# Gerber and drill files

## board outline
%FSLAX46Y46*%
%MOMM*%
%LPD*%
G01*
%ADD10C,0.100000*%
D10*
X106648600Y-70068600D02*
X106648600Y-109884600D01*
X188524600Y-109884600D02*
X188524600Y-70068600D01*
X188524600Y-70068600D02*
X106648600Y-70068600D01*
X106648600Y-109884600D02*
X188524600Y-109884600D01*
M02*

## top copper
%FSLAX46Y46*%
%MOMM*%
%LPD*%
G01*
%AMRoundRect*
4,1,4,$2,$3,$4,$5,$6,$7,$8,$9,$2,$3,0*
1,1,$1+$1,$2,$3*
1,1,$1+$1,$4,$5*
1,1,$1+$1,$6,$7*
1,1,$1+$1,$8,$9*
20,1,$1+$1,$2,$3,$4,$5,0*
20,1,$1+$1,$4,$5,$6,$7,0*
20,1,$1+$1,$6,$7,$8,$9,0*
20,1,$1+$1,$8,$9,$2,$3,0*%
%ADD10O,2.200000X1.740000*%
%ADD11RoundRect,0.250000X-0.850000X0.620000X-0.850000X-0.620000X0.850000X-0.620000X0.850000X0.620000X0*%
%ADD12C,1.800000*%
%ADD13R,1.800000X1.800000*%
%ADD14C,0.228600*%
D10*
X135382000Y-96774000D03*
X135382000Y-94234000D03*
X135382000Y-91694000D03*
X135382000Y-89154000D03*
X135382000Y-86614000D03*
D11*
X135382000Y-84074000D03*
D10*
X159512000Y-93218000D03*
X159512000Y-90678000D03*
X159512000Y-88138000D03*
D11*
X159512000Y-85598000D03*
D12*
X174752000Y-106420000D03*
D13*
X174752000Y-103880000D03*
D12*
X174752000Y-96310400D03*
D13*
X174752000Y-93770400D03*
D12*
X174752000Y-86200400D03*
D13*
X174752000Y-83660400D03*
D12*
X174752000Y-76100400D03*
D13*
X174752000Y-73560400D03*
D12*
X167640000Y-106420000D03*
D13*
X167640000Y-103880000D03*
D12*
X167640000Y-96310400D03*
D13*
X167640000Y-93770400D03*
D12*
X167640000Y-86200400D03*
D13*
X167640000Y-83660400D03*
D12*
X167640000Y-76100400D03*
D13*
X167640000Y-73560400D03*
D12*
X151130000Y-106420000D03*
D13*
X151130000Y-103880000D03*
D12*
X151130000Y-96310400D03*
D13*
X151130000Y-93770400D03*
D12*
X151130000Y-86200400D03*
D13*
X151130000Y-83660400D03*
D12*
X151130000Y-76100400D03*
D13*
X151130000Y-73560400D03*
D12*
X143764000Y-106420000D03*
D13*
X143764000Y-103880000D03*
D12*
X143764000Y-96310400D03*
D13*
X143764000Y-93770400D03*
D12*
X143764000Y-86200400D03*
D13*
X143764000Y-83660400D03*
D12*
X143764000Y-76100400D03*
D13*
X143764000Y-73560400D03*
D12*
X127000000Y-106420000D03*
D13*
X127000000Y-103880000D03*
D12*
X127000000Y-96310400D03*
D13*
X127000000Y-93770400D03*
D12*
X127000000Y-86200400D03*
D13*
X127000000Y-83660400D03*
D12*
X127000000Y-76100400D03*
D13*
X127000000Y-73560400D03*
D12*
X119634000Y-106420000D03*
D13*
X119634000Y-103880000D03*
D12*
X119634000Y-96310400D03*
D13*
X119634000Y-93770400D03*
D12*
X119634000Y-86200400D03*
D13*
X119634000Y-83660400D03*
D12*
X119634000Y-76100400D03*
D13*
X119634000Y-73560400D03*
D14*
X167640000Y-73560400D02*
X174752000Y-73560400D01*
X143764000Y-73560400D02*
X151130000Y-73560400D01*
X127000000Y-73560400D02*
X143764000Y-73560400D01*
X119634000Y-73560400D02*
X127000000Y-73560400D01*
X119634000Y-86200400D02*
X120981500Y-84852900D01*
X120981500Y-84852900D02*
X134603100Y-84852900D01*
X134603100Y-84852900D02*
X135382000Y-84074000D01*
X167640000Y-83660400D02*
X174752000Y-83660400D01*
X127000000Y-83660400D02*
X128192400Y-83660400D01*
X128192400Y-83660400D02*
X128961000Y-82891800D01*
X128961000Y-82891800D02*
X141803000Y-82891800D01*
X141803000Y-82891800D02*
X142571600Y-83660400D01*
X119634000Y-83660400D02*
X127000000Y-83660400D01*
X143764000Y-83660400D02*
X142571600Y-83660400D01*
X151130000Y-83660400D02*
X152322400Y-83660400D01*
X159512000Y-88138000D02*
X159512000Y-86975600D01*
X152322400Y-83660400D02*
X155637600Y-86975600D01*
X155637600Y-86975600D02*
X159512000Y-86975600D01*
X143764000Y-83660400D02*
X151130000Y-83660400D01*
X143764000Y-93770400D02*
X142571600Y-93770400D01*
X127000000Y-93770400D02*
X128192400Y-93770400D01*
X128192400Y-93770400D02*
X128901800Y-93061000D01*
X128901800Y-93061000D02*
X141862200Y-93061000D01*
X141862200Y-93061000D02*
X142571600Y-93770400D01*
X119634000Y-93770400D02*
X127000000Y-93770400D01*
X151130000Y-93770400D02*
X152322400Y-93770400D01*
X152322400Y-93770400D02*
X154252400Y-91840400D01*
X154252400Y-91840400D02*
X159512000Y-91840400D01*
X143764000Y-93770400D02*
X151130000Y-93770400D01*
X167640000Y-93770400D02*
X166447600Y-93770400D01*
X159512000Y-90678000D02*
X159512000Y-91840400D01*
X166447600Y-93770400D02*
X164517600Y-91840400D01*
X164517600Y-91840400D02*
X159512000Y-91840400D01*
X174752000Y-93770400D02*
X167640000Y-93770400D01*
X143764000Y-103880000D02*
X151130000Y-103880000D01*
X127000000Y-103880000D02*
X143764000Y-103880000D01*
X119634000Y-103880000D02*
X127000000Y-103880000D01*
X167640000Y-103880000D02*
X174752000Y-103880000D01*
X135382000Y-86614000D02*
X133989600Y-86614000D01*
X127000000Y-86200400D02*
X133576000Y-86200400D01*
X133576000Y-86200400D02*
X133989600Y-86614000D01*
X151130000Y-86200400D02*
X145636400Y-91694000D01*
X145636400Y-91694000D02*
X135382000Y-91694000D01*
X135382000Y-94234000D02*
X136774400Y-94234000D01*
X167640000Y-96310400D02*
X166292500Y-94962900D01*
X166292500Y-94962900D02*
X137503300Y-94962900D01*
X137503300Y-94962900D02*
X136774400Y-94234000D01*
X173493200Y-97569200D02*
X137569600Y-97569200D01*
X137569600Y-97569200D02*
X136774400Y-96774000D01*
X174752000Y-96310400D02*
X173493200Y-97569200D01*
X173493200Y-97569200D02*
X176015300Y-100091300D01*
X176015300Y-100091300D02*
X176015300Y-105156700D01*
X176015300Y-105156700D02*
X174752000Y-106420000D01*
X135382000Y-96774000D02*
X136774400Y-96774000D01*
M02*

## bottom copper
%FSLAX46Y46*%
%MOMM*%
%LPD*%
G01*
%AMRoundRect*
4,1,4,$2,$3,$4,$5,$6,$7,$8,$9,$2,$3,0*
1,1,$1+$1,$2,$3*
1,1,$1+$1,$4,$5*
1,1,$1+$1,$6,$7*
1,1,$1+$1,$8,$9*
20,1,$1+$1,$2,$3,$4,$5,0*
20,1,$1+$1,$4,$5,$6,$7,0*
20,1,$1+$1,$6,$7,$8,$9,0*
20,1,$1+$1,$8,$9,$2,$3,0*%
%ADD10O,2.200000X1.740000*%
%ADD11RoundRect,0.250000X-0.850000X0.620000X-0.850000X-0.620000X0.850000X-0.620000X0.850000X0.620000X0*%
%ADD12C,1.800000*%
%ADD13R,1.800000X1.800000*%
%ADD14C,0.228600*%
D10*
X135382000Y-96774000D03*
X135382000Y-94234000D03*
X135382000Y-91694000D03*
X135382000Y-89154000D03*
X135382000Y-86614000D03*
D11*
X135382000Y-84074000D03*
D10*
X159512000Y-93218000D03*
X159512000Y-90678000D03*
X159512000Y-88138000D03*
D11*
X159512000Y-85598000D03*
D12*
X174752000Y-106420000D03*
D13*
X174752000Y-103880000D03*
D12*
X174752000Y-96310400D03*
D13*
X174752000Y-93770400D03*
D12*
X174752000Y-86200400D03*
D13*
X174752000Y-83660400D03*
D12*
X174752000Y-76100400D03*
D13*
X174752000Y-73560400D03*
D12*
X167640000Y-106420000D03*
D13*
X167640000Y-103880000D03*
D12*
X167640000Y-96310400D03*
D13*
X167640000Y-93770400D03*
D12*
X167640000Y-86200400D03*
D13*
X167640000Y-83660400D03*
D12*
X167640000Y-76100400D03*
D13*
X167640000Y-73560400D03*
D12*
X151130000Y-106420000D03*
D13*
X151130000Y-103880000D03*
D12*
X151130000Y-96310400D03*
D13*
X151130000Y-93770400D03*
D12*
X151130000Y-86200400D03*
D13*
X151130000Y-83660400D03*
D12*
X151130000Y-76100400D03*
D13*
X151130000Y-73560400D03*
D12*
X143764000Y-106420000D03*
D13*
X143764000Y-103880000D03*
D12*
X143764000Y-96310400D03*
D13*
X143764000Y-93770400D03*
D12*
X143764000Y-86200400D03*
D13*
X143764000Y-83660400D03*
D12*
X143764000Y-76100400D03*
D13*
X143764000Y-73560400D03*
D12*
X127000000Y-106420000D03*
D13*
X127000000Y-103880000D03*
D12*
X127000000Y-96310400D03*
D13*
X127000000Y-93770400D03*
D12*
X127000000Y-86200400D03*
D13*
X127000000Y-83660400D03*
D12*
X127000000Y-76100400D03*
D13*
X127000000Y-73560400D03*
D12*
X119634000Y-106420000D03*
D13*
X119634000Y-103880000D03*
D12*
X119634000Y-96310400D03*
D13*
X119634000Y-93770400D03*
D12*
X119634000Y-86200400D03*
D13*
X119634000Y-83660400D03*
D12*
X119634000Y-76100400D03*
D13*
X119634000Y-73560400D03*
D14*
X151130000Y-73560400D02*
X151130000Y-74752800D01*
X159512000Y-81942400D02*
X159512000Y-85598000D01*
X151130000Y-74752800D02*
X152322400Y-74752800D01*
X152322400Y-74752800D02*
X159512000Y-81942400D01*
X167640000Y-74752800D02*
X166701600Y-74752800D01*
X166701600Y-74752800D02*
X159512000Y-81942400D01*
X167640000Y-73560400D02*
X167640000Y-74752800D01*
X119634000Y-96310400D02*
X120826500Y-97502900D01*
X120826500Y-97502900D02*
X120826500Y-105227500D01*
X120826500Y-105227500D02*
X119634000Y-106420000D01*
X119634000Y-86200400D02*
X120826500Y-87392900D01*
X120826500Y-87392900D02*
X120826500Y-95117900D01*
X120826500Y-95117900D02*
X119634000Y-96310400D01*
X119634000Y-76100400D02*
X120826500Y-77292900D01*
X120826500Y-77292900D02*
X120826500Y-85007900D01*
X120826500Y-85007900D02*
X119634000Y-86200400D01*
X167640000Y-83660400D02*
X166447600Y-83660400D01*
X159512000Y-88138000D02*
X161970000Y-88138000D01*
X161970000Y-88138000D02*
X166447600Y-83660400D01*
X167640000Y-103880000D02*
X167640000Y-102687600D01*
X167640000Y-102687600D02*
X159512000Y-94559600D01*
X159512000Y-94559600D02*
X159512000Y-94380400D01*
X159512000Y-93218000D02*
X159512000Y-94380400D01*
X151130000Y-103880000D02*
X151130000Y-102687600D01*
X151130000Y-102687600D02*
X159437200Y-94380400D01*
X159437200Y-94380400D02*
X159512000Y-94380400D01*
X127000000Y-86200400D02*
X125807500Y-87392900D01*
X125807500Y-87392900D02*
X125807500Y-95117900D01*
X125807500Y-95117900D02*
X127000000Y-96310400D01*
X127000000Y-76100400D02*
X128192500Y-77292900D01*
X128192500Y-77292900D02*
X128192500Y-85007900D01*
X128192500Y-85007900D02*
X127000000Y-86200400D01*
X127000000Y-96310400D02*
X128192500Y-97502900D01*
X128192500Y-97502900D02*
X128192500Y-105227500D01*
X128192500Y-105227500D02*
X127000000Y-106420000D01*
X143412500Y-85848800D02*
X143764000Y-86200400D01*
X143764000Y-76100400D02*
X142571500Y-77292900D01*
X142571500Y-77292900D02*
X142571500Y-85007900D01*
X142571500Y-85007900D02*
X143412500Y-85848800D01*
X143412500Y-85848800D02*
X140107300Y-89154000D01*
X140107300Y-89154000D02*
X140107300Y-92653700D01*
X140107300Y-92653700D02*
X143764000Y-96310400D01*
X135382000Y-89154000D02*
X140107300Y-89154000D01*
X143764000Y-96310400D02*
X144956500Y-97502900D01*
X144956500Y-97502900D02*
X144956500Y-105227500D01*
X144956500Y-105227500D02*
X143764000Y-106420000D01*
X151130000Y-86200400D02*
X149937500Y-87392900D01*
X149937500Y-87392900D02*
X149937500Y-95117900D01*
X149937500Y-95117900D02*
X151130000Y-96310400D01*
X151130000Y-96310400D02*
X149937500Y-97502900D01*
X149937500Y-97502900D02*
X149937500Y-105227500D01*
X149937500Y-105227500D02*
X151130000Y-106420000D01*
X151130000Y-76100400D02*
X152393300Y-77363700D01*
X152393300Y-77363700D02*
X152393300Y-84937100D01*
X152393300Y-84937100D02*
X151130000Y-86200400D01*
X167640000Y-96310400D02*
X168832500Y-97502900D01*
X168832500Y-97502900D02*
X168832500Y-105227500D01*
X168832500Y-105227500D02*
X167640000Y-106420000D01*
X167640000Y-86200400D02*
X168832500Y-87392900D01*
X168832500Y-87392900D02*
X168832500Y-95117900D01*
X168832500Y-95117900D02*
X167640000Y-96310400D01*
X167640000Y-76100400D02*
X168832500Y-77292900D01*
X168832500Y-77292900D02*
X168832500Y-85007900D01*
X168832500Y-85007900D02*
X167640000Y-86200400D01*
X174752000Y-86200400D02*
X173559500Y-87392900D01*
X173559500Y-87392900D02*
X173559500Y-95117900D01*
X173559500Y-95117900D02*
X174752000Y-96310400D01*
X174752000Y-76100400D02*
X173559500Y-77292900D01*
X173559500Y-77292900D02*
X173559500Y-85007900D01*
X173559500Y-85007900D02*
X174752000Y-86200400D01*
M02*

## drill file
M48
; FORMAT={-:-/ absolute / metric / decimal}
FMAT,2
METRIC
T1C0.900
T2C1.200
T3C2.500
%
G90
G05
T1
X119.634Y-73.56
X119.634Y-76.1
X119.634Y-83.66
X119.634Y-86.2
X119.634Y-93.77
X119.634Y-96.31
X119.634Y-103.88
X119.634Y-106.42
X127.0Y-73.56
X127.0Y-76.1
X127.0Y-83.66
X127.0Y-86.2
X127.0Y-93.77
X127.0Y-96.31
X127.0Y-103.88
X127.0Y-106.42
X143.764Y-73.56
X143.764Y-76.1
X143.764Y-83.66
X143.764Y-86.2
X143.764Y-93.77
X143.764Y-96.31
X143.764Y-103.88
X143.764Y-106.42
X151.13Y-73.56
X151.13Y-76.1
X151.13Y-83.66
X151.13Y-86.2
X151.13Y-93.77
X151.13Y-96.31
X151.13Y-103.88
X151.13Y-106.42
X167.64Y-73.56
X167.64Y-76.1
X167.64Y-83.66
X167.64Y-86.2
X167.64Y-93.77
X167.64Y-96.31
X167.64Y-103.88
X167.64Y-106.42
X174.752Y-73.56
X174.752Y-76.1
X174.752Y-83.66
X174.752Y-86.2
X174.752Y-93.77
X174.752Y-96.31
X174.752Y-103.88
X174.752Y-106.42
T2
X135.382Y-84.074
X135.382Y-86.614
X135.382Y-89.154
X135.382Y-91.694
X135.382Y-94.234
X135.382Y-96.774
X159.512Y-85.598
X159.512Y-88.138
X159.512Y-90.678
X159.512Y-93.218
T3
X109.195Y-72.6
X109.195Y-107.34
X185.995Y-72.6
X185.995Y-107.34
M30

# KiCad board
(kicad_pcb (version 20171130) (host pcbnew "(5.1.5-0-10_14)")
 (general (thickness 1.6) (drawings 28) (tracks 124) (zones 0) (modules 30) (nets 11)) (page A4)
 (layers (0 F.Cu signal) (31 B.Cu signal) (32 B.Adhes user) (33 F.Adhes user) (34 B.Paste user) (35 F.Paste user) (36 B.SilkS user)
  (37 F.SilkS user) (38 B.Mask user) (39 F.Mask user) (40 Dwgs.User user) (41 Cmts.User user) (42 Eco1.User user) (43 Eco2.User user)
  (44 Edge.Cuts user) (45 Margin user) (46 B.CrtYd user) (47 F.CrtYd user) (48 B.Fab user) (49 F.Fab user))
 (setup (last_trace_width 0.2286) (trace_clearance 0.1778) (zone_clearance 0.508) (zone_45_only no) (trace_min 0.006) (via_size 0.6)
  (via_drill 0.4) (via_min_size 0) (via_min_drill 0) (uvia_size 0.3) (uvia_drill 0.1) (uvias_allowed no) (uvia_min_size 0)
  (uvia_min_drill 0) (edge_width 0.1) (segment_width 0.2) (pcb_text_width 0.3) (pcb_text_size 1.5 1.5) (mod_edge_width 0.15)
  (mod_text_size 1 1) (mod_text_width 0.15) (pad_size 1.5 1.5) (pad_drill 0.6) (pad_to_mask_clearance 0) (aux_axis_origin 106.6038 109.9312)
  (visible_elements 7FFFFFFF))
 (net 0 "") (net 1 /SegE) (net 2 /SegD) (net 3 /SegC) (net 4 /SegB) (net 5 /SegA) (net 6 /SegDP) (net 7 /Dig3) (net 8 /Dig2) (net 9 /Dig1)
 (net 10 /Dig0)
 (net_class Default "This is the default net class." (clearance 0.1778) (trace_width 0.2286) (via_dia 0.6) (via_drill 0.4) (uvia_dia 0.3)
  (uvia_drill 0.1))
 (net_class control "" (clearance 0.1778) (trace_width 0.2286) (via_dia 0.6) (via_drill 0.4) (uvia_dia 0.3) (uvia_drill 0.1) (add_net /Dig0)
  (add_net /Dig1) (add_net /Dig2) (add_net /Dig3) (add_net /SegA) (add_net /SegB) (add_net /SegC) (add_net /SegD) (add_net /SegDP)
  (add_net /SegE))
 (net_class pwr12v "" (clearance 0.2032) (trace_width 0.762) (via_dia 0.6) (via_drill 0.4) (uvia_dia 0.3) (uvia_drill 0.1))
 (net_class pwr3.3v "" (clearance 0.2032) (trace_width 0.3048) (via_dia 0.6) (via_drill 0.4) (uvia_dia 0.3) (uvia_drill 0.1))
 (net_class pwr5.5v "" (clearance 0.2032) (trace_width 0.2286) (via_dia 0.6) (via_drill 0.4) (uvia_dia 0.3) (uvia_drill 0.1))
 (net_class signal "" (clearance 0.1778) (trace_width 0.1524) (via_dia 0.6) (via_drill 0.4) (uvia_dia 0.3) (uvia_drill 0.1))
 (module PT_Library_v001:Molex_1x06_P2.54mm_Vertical (layer B.Cu) (at 135.382 84.074 270)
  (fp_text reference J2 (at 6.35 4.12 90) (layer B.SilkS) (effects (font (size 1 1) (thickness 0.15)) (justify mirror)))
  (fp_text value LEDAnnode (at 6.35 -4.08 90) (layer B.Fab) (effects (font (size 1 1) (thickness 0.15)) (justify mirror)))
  (pad 6 thru_hole oval (at 12.7 0 270) (size 1.74 2.2) (drill 1.2) (layers *.Cu *.Mask) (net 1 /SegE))
  (pad 5 thru_hole oval (at 10.16 0 270) (size 1.74 2.2) (drill 1.2) (layers *.Cu *.Mask) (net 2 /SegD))
  (pad 4 thru_hole oval (at 7.62 0 270) (size 1.74 2.2) (drill 1.2) (layers *.Cu *.Mask) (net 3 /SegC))
  (pad 3 thru_hole oval (at 5.08 0 270) (size 1.74 2.2) (drill 1.2) (layers *.Cu *.Mask) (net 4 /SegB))
  (pad 2 thru_hole oval (at 2.54 0 270) (size 1.74 2.2) (drill 1.2) (layers *.Cu *.Mask) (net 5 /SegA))
  (pad 1 thru_hole roundrect (at 0 0 270) (size 1.74 2.2) (drill 1.2) (layers *.Cu *.Mask) (roundrect_rratio 0.143678) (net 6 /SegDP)))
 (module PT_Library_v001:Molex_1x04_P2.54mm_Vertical (layer B.Cu) (at 159.512 85.598 270)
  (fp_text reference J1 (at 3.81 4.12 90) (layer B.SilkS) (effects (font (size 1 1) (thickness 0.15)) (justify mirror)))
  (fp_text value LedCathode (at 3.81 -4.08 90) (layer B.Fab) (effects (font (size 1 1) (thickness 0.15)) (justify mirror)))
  (pad 4 thru_hole oval (at 7.62 0 270) (size 1.74 2.2) (drill 1.2) (layers *.Cu *.Mask) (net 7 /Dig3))
  (pad 3 thru_hole oval (at 5.08 0 270) (size 1.74 2.2) (drill 1.2) (layers *.Cu *.Mask) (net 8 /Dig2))
  (pad 2 thru_hole oval (at 2.54 0 270) (size 1.74 2.2) (drill 1.2) (layers *.Cu *.Mask) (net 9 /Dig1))
  (pad 1 thru_hole roundrect (at 0 0 270) (size 1.74 2.2) (drill 1.2) (layers *.Cu *.Mask) (roundrect_rratio 0.143678) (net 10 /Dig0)))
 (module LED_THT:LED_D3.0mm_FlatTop (layer F.Cu) (at 174.752 103.88 270)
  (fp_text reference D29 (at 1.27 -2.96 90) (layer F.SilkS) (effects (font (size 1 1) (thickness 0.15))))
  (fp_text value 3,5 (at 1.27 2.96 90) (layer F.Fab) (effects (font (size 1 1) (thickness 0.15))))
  (pad 2 thru_hole circle (at 2.54 0 270) (size 1.8 1.8) (drill 0.9) (layers *.Cu *.Mask) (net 1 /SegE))
  (pad 1 thru_hole rect (at 0 0 270) (size 1.8 1.8) (drill 0.9) (layers *.Cu *.Mask) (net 7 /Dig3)))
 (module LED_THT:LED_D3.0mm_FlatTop (layer F.Cu) (at 174.752 93.7704 270)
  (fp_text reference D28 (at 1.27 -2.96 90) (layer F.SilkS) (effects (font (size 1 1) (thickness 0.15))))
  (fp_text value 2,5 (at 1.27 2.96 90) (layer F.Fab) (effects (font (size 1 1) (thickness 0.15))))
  (pad 2 thru_hole circle (at 2.54 0 270) (size 1.8 1.8) (drill 0.9) (layers *.Cu *.Mask) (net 1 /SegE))
  (pad 1 thru_hole rect (at 0 0 270) (size 1.8 1.8) (drill 0.9) (layers *.Cu *.Mask) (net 8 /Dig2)))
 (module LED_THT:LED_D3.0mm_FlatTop (layer F.Cu) (at 174.752 83.6604 270)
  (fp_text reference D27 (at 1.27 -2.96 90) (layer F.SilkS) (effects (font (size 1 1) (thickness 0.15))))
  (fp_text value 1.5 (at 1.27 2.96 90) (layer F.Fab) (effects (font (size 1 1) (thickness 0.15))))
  (pad 2 thru_hole circle (at 2.54 0 270) (size 1.8 1.8) (drill 0.9) (layers *.Cu *.Mask) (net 1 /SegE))
  (pad 1 thru_hole rect (at 0 0 270) (size 1.8 1.8) (drill 0.9) (layers *.Cu *.Mask) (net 9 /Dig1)))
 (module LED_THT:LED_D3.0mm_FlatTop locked (layer F.Cu) (at 174.752 73.5604 270)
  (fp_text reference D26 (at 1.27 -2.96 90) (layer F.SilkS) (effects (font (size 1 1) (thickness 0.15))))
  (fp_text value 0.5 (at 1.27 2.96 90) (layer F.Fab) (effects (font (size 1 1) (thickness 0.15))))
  (pad 2 thru_hole circle (at 2.54 0 270) (size 1.8 1.8) (drill 0.9) (layers *.Cu *.Mask) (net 1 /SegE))
  (pad 1 thru_hole rect (at 0 0 270) (size 1.8 1.8) (drill 0.9) (layers *.Cu *.Mask) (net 10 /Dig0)))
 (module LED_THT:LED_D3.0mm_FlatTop (layer F.Cu) (at 167.64 103.88 270)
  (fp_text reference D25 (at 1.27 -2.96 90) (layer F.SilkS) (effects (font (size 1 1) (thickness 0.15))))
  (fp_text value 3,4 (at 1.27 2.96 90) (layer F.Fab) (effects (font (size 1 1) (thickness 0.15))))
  (pad 2 thru_hole circle (at 2.54 0 270) (size 1.8 1.8) (drill 0.9) (layers *.Cu *.Mask) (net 2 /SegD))
  (pad 1 thru_hole rect (at 0 0 270) (size 1.8 1.8) (drill 0.9) (layers *.Cu *.Mask) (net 7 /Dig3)))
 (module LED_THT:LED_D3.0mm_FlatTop (layer F.Cu) (at 167.64 93.7704 270)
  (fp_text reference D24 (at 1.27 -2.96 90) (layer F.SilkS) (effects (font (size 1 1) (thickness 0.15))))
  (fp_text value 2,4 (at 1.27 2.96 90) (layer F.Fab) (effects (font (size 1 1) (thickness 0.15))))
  (pad 2 thru_hole circle (at 2.54 0 270) (size 1.8 1.8) (drill 0.9) (layers *.Cu *.Mask) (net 2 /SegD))
  (pad 1 thru_hole rect (at 0 0 270) (size 1.8 1.8) (drill 0.9) (layers *.Cu *.Mask) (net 8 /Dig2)))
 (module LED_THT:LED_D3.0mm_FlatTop (layer F.Cu) (at 167.64 83.6604 270)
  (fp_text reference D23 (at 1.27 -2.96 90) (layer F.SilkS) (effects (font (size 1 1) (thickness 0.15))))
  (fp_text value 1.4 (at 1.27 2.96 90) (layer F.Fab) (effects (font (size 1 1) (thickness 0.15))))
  (pad 2 thru_hole circle (at 2.54 0 270) (size 1.8 1.8) (drill 0.9) (layers *.Cu *.Mask) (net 2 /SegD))
  (pad 1 thru_hole rect (at 0 0 270) (size 1.8 1.8) (drill 0.9) (layers *.Cu *.Mask) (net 9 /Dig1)))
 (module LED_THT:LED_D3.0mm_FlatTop (layer F.Cu) (at 167.64 73.5604 270)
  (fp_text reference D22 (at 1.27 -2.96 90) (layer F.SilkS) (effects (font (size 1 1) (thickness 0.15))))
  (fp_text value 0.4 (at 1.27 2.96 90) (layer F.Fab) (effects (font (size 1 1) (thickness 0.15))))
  (pad 2 thru_hole circle (at 2.54 0 270) (size 1.8 1.8) (drill 0.9) (layers *.Cu *.Mask) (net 2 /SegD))
  (pad 1 thru_hole rect (at 0 0 270) (size 1.8 1.8) (drill 0.9) (layers *.Cu *.Mask) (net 10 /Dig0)))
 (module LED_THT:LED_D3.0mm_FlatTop (layer F.Cu) (at 151.13 103.88 270)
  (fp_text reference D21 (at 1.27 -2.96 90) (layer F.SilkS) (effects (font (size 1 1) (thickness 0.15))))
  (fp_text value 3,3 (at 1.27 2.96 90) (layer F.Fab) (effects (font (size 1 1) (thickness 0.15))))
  (pad 2 thru_hole circle (at 2.54 0 270) (size 1.8 1.8) (drill 0.9) (layers *.Cu *.Mask) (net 3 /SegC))
  (pad 1 thru_hole rect (at 0 0 270) (size 1.8 1.8) (drill 0.9) (layers *.Cu *.Mask) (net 7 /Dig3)))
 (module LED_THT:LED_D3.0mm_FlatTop (layer F.Cu) (at 151.13 93.7704 270)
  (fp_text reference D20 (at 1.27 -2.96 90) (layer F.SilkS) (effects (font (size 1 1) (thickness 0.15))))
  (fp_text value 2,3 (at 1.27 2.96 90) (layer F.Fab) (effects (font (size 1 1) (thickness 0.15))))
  (pad 2 thru_hole circle (at 2.54 0 270) (size 1.8 1.8) (drill 0.9) (layers *.Cu *.Mask) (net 3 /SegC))
  (pad 1 thru_hole rect (at 0 0 270) (size 1.8 1.8) (drill 0.9) (layers *.Cu *.Mask) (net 8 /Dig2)))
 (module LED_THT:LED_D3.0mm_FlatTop (layer F.Cu) (at 151.13 83.6604 270)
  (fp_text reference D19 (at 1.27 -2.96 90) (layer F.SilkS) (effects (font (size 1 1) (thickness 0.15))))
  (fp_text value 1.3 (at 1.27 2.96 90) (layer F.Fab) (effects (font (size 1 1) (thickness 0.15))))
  (pad 2 thru_hole circle (at 2.54 0 270) (size 1.8 1.8) (drill 0.9) (layers *.Cu *.Mask) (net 3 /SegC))
  (pad 1 thru_hole rect (at 0 0 270) (size 1.8 1.8) (drill 0.9) (layers *.Cu *.Mask) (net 9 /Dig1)))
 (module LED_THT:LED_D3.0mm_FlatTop (layer F.Cu) (at 151.13 73.5604 270)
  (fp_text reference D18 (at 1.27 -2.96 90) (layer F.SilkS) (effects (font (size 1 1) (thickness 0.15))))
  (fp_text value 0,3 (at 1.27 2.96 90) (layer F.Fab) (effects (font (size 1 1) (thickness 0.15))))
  (pad 2 thru_hole circle (at 2.54 0 270) (size 1.8 1.8) (drill 0.9) (layers *.Cu *.Mask) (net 3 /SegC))
  (pad 1 thru_hole rect (at 0 0 270) (size 1.8 1.8) (drill 0.9) (layers *.Cu *.Mask) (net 10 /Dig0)))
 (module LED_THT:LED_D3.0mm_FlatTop (layer F.Cu) (at 143.764 103.88 270)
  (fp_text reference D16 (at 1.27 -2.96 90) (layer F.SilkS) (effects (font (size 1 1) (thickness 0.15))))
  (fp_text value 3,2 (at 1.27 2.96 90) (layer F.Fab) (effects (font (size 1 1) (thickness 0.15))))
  (pad 2 thru_hole circle (at 2.54 0 270) (size 1.8 1.8) (drill 0.9) (layers *.Cu *.Mask) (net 4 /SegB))
  (pad 1 thru_hole rect (at 0 0 270) (size 1.8 1.8) (drill 0.9) (layers *.Cu *.Mask) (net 7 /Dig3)))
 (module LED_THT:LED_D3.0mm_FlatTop (layer F.Cu) (at 143.764 93.7704 270)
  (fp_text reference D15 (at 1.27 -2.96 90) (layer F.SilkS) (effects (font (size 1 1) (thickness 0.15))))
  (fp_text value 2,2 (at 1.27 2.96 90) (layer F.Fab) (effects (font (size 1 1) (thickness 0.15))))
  (pad 2 thru_hole circle (at 2.54 0 270) (size 1.8 1.8) (drill 0.9) (layers *.Cu *.Mask) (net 4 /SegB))
  (pad 1 thru_hole rect (at 0 0 270) (size 1.8 1.8) (drill 0.9) (layers *.Cu *.Mask) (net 8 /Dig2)))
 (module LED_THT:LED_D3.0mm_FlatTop (layer F.Cu) (at 143.764 83.6604 270)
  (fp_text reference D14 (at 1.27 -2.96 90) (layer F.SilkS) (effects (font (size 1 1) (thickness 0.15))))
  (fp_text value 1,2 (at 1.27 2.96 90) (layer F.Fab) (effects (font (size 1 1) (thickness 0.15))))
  (pad 2 thru_hole circle (at 2.54 0 270) (size 1.8 1.8) (drill 0.9) (layers *.Cu *.Mask) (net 4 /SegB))
  (pad 1 thru_hole rect (at 0 0 270) (size 1.8 1.8) (drill 0.9) (layers *.Cu *.Mask) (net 9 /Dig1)))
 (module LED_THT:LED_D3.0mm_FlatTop (layer F.Cu) (at 143.764 73.5604 270)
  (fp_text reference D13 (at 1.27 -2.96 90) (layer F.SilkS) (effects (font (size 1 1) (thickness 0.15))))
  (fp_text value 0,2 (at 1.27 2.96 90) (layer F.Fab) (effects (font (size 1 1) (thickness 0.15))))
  (pad 2 thru_hole circle (at 2.54 0 270) (size 1.8 1.8) (drill 0.9) (layers *.Cu *.Mask) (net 4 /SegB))
  (pad 1 thru_hole rect (at 0 0 270) (size 1.8 1.8) (drill 0.9) (layers *.Cu *.Mask) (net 10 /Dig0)))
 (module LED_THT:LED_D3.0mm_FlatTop (layer F.Cu) (at 127 103.88 270)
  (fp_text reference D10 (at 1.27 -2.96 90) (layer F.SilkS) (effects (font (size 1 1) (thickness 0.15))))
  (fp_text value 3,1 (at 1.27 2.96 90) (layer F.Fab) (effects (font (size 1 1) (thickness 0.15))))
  (pad 2 thru_hole circle (at 2.54 0 270) (size 1.8 1.8) (drill 0.9) (layers *.Cu *.Mask) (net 5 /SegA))
  (pad 1 thru_hole rect (at 0 0 270) (size 1.8 1.8) (drill 0.9) (layers *.Cu *.Mask) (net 7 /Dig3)))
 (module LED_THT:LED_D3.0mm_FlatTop (layer F.Cu) (at 127 93.7704 270)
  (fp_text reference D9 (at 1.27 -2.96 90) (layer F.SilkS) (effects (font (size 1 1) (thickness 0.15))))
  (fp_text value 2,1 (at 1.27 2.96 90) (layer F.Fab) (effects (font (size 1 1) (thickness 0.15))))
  (pad 2 thru_hole circle (at 2.54 0 270) (size 1.8 1.8) (drill 0.9) (layers *.Cu *.Mask) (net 5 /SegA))
  (pad 1 thru_hole rect (at 0 0 270) (size 1.8 1.8) (drill 0.9) (layers *.Cu *.Mask) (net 8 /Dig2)))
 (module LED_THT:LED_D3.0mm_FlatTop (layer F.Cu) (at 127 83.6604 270)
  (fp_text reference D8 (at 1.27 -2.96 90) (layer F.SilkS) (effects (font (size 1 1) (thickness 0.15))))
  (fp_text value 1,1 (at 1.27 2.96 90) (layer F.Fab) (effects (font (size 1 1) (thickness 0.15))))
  (pad 2 thru_hole circle (at 2.54 0 270) (size 1.8 1.8) (drill 0.9) (layers *.Cu *.Mask) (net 5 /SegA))
  (pad 1 thru_hole rect (at 0 0 270) (size 1.8 1.8) (drill 0.9) (layers *.Cu *.Mask) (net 9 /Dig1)))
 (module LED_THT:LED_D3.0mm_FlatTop (layer F.Cu) (at 127 73.5604 270)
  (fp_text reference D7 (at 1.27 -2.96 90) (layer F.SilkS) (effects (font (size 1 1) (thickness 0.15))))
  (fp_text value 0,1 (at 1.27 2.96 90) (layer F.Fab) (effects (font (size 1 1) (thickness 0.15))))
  (pad 2 thru_hole circle (at 2.54 0 270) (size 1.8 1.8) (drill 0.9) (layers *.Cu *.Mask) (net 5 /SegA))
  (pad 1 thru_hole rect (at 0 0 270) (size 1.8 1.8) (drill 0.9) (layers *.Cu *.Mask) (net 10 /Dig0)))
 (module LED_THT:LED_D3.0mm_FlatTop (layer F.Cu) (at 119.634 103.88 270)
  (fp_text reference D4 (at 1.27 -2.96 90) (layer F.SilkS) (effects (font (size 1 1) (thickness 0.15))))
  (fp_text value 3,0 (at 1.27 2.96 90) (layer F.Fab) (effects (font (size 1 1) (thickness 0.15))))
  (pad 2 thru_hole circle (at 2.54 0 270) (size 1.8 1.8) (drill 0.9) (layers *.Cu *.Mask) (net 6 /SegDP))
  (pad 1 thru_hole rect (at 0 0 270) (size 1.8 1.8) (drill 0.9) (layers *.Cu *.Mask) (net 7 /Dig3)))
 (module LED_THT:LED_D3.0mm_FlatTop (layer F.Cu) (at 119.634 93.7704 270)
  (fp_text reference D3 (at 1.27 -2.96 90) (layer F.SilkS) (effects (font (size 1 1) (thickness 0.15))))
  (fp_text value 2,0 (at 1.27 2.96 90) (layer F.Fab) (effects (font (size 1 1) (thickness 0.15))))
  (pad 2 thru_hole circle (at 2.54 0 270) (size 1.8 1.8) (drill 0.9) (layers *.Cu *.Mask) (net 6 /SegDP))
  (pad 1 thru_hole rect (at 0 0 270) (size 1.8 1.8) (drill 0.9) (layers *.Cu *.Mask) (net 8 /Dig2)))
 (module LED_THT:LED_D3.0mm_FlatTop (layer F.Cu) (at 119.634 83.6604 270)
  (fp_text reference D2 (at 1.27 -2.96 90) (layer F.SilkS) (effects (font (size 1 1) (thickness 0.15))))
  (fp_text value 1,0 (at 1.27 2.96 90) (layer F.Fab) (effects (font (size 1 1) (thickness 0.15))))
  (pad 2 thru_hole circle (at 2.54 0 270) (size 1.8 1.8) (drill 0.9) (layers *.Cu *.Mask) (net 6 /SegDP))
  (pad 1 thru_hole rect (at 0 0 270) (size 1.8 1.8) (drill 0.9) (layers *.Cu *.Mask) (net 9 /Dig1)))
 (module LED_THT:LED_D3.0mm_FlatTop (layer F.Cu) (at 119.634 73.5604 270)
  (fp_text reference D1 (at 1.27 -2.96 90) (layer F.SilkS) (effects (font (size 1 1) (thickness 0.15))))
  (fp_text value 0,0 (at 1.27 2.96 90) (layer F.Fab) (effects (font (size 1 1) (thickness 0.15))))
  (pad 2 thru_hole circle (at 2.54 0 270) (size 1.8 1.8) (drill 0.9) (layers *.Cu *.Mask) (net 6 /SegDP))
  (pad 1 thru_hole rect (at 0 0 270) (size 1.8 1.8) (drill 0.9) (layers *.Cu *.Mask) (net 10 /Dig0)))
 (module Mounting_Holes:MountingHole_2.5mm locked (layer F.Cu) (at 109.195 72.6004)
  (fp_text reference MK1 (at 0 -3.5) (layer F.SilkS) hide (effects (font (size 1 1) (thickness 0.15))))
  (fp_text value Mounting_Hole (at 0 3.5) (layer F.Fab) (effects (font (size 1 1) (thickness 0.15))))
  (pad 1 np_thru_hole circle (at 0 0) (size 2.5 2.5) (drill 2.5) (layers *.Cu *.Mask)))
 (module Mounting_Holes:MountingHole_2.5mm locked (layer F.Cu) (at 185.995 72.6004)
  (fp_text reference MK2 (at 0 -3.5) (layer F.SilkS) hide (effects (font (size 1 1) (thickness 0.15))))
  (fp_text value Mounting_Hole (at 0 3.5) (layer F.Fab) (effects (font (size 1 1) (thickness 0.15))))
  (pad 1 np_thru_hole circle (at 0 0) (size 2.5 2.5) (drill 2.5) (layers *.Cu *.Mask)))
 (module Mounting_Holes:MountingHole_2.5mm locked (layer F.Cu) (at 109.195 107.34)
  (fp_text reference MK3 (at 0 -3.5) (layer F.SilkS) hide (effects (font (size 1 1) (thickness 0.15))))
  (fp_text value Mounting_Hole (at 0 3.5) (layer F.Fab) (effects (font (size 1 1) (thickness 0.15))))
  (pad 1 np_thru_hole circle (at 0 0) (size 2.5 2.5) (drill 2.5) (layers *.Cu *.Mask)))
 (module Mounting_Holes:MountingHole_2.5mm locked (layer F.Cu) (at 185.995 107.34)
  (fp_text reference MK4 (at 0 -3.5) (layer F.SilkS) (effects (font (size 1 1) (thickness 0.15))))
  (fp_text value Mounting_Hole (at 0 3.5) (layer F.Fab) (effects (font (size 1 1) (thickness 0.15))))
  (pad 1 np_thru_hole circle (at 0 0) (size 2.5 2.5) (drill 2.5) (layers *.Cu *.Mask)))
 (gr_line (start 106.6486 70.0686) (end 106.6486 109.8846) (layer Edge.Cuts) (width 0.1))
 (gr_line (start 188.5246 109.8846) (end 188.5246 70.0686) (layer Edge.Cuts) (width 0.1))
 (gr_line (start 188.5246 70.0686) (end 106.6486 70.0686) (layer Edge.Cuts) (width 0.1))
 (gr_line (start 106.6486 109.8846) (end 188.5246 109.8846) (layer Edge.Cuts) (width 0.1))
 (segment (start 151.13 73.5604) (end 151.13 74.7528) (width 0.2286) (layer B.Cu) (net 10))
 (segment (start 159.512 81.9424) (end 159.512 85.598) (width 0.2286) (layer B.Cu) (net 10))
 (segment (start 151.13 74.7528) (end 152.3224 74.7528) (width 0.2286) (layer B.Cu) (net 10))
 (segment (start 152.3224 74.7528) (end 159.512 81.9424) (width 0.2286) (layer B.Cu) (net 10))
 (segment (start 167.64 74.7528) (end 166.7016 74.7528) (width 0.2286) (layer B.Cu) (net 10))
 (segment (start 166.7016 74.7528) (end 159.512 81.9424) (width 0.2286) (layer B.Cu) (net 10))
 (segment (start 167.64 73.5604) (end 167.64 74.7528) (width 0.2286) (layer B.Cu) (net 10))
 (segment (start 167.64 73.5604) (end 174.752 73.5604) (width 0.2286) (layer F.Cu) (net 10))
 (segment (start 143.764 73.5604) (end 151.13 73.5604) (width 0.2286) (layer F.Cu) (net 10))
 (segment (start 127 73.5604) (end 143.764 73.5604) (width 0.2286) (layer F.Cu) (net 10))
 (segment (start 119.634 73.5604) (end 127 73.5604) (width 0.2286) (layer F.Cu) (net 10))
 (segment (start 119.634 86.2004) (end 120.9815 84.8529) (width 0.2286) (layer F.Cu) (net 6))
 (segment (start 120.9815 84.8529) (end 134.6031 84.8529) (width 0.2286) (layer F.Cu) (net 6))
 (segment (start 134.6031 84.8529) (end 135.382 84.074) (width 0.2286) (layer F.Cu) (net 6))
 (segment (start 119.634 96.3104) (end 120.8265 97.5029) (width 0.2286) (layer B.Cu) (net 6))
 (segment (start 120.8265 97.5029) (end 120.8265 105.2275) (width 0.2286) (layer B.Cu) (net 6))
 (segment (start 120.8265 105.2275) (end 119.634 106.42) (width 0.2286) (layer B.Cu) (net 6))
 (segment (start 119.634 86.2004) (end 120.8265 87.3929) (width 0.2286) (layer B.Cu) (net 6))
 (segment (start 120.8265 87.3929) (end 120.8265 95.1179) (width 0.2286) (layer B.Cu) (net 6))
 (segment (start 120.8265 95.1179) (end 119.634 96.3104) (width 0.2286) (layer B.Cu) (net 6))
 (segment (start 119.634 76.1004) (end 120.8265 77.2929) (width 0.2286) (layer B.Cu) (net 6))
 (segment (start 120.8265 77.2929) (end 120.8265 85.0079) (width 0.2286) (layer B.Cu) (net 6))
 (segment (start 120.8265 85.0079) (end 119.634 86.2004) (width 0.2286) (layer B.Cu) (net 6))
 (segment (start 167.64 83.6604) (end 174.752 83.6604) (width 0.2286) (layer F.Cu) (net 9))
 (segment (start 167.64 83.6604) (end 166.4476 83.6604) (width 0.2286) (layer B.Cu) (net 9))
 (segment (start 159.512 88.138) (end 161.97 88.138) (width 0.2286) (layer B.Cu) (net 9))
 (segment (start 161.97 88.138) (end 166.4476 83.6604) (width 0.2286) (layer B.Cu) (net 9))
 (segment (start 127 83.6604) (end 128.1924 83.6604) (width 0.2286) (layer F.Cu) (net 9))
 (segment (start 128.1924 83.6604) (end 128.961 82.8918) (width 0.2286) (layer F.Cu) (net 9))
 (segment (start 128.961 82.8918) (end 141.803 82.8918) (width 0.2286) (layer F.Cu) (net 9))
 (segment (start 141.803 82.8918) (end 142.5716 83.6604) (width 0.2286) (layer F.Cu) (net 9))
 (segment (start 119.634 83.6604) (end 127 83.6604) (width 0.2286) (layer F.Cu) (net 9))
 (segment (start 143.764 83.6604) (end 142.5716 83.6604) (width 0.2286) (layer F.Cu) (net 9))
 (segment (start 151.13 83.6604) (end 152.3224 83.6604) (width 0.2286) (layer F.Cu) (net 9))
 (segment (start 159.512 88.138) (end 159.512 86.9756) (width 0.2286) (layer F.Cu) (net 9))
 (segment (start 152.3224 83.6604) (end 155.6376 86.9756) (width 0.2286) (layer F.Cu) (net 9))
 (segment (start 155.6376 86.9756) (end 159.512 86.9756) (width 0.2286) (layer F.Cu) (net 9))
 (segment (start 143.764 83.6604) (end 151.13 83.6604) (width 0.2286) (layer F.Cu) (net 9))
 (segment (start 143.764 93.7704) (end 142.5716 93.7704) (width 0.2286) (layer F.Cu) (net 8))
 (segment (start 127 93.7704) (end 128.1924 93.7704) (width 0.2286) (layer F.Cu) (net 8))
 (segment (start 128.1924 93.7704) (end 128.9018 93.061) (width 0.2286) (layer F.Cu) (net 8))
 (segment (start 128.9018 93.061) (end 141.8622 93.061) (width 0.2286) (layer F.Cu) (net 8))
 (segment (start 141.8622 93.061) (end 142.5716 93.7704) (width 0.2286) (layer F.Cu) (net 8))
 (segment (start 119.634 93.7704) (end 127 93.7704) (width 0.2286) (layer F.Cu) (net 8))
 (segment (start 151.13 93.7704) (end 152.3224 93.7704) (width 0.2286) (layer F.Cu) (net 8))
 (segment (start 152.3224 93.7704) (end 154.2524 91.8404) (width 0.2286) (layer F.Cu) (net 8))
 (segment (start 154.2524 91.8404) (end 159.512 91.8404) (width 0.2286) (layer F.Cu) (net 8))
 (segment (start 143.764 93.7704) (end 151.13 93.7704) (width 0.2286) (layer F.Cu) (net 8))
 (segment (start 167.64 93.7704) (end 166.4476 93.7704) (width 0.2286) (layer F.Cu) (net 8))
 (segment (start 159.512 90.678) (end 159.512 91.8404) (width 0.2286) (layer F.Cu) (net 8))
 (segment (start 166.4476 93.7704) (end 164.5176 91.8404) (width 0.2286) (layer F.Cu) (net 8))
 (segment (start 164.5176 91.8404) (end 159.512 91.8404) (width 0.2286) (layer F.Cu) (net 8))
 (segment (start 174.752 93.7704) (end 167.64 93.7704) (width 0.2286) (layer F.Cu) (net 8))
 (segment (start 143.764 103.88) (end 151.13 103.88) (width 0.2286) (layer F.Cu) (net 7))
 (segment (start 127 103.88) (end 143.764 103.88) (width 0.2286) (layer F.Cu) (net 7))
 (segment (start 119.634 103.88) (end 127 103.88) (width 0.2286) (layer F.Cu) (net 7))
 (segment (start 167.64 103.88) (end 167.64 102.6876) (width 0.2286) (layer B.Cu) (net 7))
 (segment (start 167.64 102.6876) (end 159.512 94.5596) (width 0.2286) (layer B.Cu) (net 7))
 (segment (start 159.512 94.5596) (end 159.512 94.3804) (width 0.2286) (layer B.Cu) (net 7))
 (segment (start 167.64 103.88) (end 174.752 103.88) (width 0.2286) (layer F.Cu) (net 7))
 (segment (start 159.512 93.218) (end 159.512 94.3804) (width 0.2286) (layer B.Cu) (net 7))
 (segment (start 151.13 103.88) (end 151.13 102.6876) (width 0.2286) (layer B.Cu) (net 7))
 (segment (start 151.13 102.6876) (end 159.4372 94.3804) (width 0.2286) (layer B.Cu) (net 7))
 (segment (start 159.4372 94.3804) (end 159.512 94.3804) (width 0.2286) (layer B.Cu) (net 7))
 (segment (start 127 86.2004) (end 125.8075 87.3929) (width 0.2286) (layer B.Cu) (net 5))
 (segment (start 125.8075 87.3929) (end 125.8075 95.1179) (width 0.2286) (layer B.Cu) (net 5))
 (segment (start 125.8075 95.1179) (end 127 96.3104) (width 0.2286) (layer B.Cu) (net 5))
 (segment (start 127 76.1004) (end 128.1925 77.2929) (width 0.2286) (layer B.Cu) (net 5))
 (segment (start 128.1925 77.2929) (end 128.1925 85.0079) (width 0.2286) (layer B.Cu) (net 5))
 (segment (start 128.1925 85.0079) (end 127 86.2004) (width 0.2286) (layer B.Cu) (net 5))
 (segment (start 127 96.3104) (end 128.1925 97.5029) (width 0.2286) (layer B.Cu) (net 5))
 (segment (start 128.1925 97.5029) (end 128.1925 105.2275) (width 0.2286) (layer B.Cu) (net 5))
 (segment (start 128.1925 105.2275) (end 127 106.42) (width 0.2286) (layer B.Cu) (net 5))
 (segment (start 135.382 86.614) (end 133.9896 86.614) (width 0.2286) (layer F.Cu) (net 5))
 (segment (start 127 86.2004) (end 133.576 86.2004) (width 0.2286) (layer F.Cu) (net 5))
 (segment (start 133.576 86.2004) (end 133.9896 86.614) (width 0.2286) (layer F.Cu) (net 5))
 (segment (start 143.4125 85.8488) (end 143.764 86.2004) (width 0.2286) (layer B.Cu) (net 4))
 (segment (start 143.764 76.1004) (end 142.5715 77.2929) (width 0.2286) (layer B.Cu) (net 4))
 (segment (start 142.5715 77.2929) (end 142.5715 85.0079) (width 0.2286) (layer B.Cu) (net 4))
 (segment (start 142.5715 85.0079) (end 143.4125 85.8488) (width 0.2286) (layer B.Cu) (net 4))
 (segment (start 143.4125 85.8488) (end 140.1073 89.154) (width 0.2286) (layer B.Cu) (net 4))
 (segment (start 140.1073 89.154) (end 140.1073 92.6537) (width 0.2286) (layer B.Cu) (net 4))
 (segment (start 140.1073 92.6537) (end 143.764 96.3104) (width 0.2286) (layer B.Cu) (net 4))
 (segment (start 135.382 89.154) (end 140.1073 89.154) (width 0.2286) (layer B.Cu) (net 4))
 (segment (start 143.764 96.3104) (end 144.9565 97.5029) (width 0.2286) (layer B.Cu) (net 4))
 (segment (start 144.9565 97.5029) (end 144.9565 105.2275) (width 0.2286) (layer B.Cu) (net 4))
 (segment (start 144.9565 105.2275) (end 143.764 106.42) (width 0.2286) (layer B.Cu) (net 4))
 (segment (start 151.13 86.2004) (end 145.6364 91.694) (width 0.2286) (layer F.Cu) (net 3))
 (segment (start 145.6364 91.694) (end 135.382 91.694) (width 0.2286) (layer F.Cu) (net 3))
 (segment (start 151.13 86.2004) (end 149.9375 87.3929) (width 0.2286) (layer B.Cu) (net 3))
 (segment (start 149.9375 87.3929) (end 149.9375 95.1179) (width 0.2286) (layer B.Cu) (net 3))
 (segment (start 149.9375 95.1179) (end 151.13 96.3104) (width 0.2286) (layer B.Cu) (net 3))
 (segment (start 151.13 96.3104) (end 149.9375 97.5029) (width 0.2286) (layer B.Cu) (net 3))
 (segment (start 149.9375 97.5029) (end 149.9375 105.2275) (width 0.2286) (layer B.Cu) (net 3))
 (segment (start 149.9375 105.2275) (end 151.13 106.42) (width 0.2286) (layer B.Cu) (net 3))
 (segment (start 151.13 76.1004) (end 152.3933 77.3637) (width 0.2286) (layer B.Cu) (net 3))
 (segment (start 152.3933 77.3637) (end 152.3933 84.9371) (width 0.2286) (layer B.Cu) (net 3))
 (segment (start 152.3933 84.9371) (end 151.13 86.2004) (width 0.2286) (layer B.Cu) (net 3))
 (segment (start 135.382 94.234) (end 136.7744 94.234) (width 0.2286) (layer F.Cu) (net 2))
 (segment (start 167.64 96.3104) (end 166.2925 94.9629) (width 0.2286) (layer F.Cu) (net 2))
 (segment (start 166.2925 94.9629) (end 137.5033 94.9629) (width 0.2286) (layer F.Cu) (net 2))
 (segment (start 137.5033 94.9629) (end 136.7744 94.234) (width 0.2286) (layer F.Cu) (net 2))
 (segment (start 167.64 96.3104) (end 168.8325 97.5029) (width 0.2286) (layer B.Cu) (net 2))
 (segment (start 168.8325 97.5029) (end 168.8325 105.2275) (width 0.2286) (layer B.Cu) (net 2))
 (segment (start 168.8325 105.2275) (end 167.64 106.42) (width 0.2286) (layer B.Cu) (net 2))
 (segment (start 167.64 86.2004) (end 168.8325 87.3929) (width 0.2286) (layer B.Cu) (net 2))
 (segment (start 168.8325 87.3929) (end 168.8325 95.1179) (width 0.2286) (layer B.Cu) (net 2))
 (segment (start 168.8325 95.1179) (end 167.64 96.3104) (width 0.2286) (layer B.Cu) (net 2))
 (segment (start 167.64 76.1004) (end 168.8325 77.2929) (width 0.2286) (layer B.Cu) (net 2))
 (segment (start 168.8325 77.2929) (end 168.8325 85.0079) (width 0.2286) (layer B.Cu) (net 2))
 (segment (start 168.8325 85.0079) (end 167.64 86.2004) (width 0.2286) (layer B.Cu) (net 2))
 (segment (start 173.4932 97.5692) (end 137.5696 97.5692) (width 0.2286) (layer F.Cu) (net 1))
 (segment (start 137.5696 97.5692) (end 136.7744 96.774) (width 0.2286) (layer F.Cu) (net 1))
 (segment (start 174.752 96.3104) (end 173.4932 97.5692) (width 0.2286) (layer F.Cu) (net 1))
 (segment (start 173.4932 97.5692) (end 176.0153 100.0913) (width 0.2286) (layer F.Cu) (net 1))
 (segment (start 176.0153 100.0913) (end 176.0153 105.1567) (width 0.2286) (layer F.Cu) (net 1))
 (segment (start 176.0153 105.1567) (end 174.752 106.42) (width 0.2286) (layer F.Cu) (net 1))
 (segment (start 135.382 96.774) (end 136.7744 96.774) (width 0.2286) (layer F.Cu) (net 1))
 (segment (start 174.752 86.2004) (end 173.5595 87.3929) (width 0.2286) (layer B.Cu) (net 1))
 (segment (start 173.5595 87.3929) (end 173.5595 95.1179) (width 0.2286) (layer B.Cu) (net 1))
 (segment (start 173.5595 95.1179) (end 174.752 96.3104) (width 0.2286) (layer B.Cu) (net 1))
 (segment (start 174.752 76.1004) (end 173.5595 77.2929) (width 0.2286) (layer B.Cu) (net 1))
 (segment (start 173.5595 77.2929) (end 173.5595 85.0079) (width 0.2286) (layer B.Cu) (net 1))
 (segment (start 173.5595 85.0079) (end 174.752 86.2004) (width 0.2286) (layer B.Cu) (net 1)))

